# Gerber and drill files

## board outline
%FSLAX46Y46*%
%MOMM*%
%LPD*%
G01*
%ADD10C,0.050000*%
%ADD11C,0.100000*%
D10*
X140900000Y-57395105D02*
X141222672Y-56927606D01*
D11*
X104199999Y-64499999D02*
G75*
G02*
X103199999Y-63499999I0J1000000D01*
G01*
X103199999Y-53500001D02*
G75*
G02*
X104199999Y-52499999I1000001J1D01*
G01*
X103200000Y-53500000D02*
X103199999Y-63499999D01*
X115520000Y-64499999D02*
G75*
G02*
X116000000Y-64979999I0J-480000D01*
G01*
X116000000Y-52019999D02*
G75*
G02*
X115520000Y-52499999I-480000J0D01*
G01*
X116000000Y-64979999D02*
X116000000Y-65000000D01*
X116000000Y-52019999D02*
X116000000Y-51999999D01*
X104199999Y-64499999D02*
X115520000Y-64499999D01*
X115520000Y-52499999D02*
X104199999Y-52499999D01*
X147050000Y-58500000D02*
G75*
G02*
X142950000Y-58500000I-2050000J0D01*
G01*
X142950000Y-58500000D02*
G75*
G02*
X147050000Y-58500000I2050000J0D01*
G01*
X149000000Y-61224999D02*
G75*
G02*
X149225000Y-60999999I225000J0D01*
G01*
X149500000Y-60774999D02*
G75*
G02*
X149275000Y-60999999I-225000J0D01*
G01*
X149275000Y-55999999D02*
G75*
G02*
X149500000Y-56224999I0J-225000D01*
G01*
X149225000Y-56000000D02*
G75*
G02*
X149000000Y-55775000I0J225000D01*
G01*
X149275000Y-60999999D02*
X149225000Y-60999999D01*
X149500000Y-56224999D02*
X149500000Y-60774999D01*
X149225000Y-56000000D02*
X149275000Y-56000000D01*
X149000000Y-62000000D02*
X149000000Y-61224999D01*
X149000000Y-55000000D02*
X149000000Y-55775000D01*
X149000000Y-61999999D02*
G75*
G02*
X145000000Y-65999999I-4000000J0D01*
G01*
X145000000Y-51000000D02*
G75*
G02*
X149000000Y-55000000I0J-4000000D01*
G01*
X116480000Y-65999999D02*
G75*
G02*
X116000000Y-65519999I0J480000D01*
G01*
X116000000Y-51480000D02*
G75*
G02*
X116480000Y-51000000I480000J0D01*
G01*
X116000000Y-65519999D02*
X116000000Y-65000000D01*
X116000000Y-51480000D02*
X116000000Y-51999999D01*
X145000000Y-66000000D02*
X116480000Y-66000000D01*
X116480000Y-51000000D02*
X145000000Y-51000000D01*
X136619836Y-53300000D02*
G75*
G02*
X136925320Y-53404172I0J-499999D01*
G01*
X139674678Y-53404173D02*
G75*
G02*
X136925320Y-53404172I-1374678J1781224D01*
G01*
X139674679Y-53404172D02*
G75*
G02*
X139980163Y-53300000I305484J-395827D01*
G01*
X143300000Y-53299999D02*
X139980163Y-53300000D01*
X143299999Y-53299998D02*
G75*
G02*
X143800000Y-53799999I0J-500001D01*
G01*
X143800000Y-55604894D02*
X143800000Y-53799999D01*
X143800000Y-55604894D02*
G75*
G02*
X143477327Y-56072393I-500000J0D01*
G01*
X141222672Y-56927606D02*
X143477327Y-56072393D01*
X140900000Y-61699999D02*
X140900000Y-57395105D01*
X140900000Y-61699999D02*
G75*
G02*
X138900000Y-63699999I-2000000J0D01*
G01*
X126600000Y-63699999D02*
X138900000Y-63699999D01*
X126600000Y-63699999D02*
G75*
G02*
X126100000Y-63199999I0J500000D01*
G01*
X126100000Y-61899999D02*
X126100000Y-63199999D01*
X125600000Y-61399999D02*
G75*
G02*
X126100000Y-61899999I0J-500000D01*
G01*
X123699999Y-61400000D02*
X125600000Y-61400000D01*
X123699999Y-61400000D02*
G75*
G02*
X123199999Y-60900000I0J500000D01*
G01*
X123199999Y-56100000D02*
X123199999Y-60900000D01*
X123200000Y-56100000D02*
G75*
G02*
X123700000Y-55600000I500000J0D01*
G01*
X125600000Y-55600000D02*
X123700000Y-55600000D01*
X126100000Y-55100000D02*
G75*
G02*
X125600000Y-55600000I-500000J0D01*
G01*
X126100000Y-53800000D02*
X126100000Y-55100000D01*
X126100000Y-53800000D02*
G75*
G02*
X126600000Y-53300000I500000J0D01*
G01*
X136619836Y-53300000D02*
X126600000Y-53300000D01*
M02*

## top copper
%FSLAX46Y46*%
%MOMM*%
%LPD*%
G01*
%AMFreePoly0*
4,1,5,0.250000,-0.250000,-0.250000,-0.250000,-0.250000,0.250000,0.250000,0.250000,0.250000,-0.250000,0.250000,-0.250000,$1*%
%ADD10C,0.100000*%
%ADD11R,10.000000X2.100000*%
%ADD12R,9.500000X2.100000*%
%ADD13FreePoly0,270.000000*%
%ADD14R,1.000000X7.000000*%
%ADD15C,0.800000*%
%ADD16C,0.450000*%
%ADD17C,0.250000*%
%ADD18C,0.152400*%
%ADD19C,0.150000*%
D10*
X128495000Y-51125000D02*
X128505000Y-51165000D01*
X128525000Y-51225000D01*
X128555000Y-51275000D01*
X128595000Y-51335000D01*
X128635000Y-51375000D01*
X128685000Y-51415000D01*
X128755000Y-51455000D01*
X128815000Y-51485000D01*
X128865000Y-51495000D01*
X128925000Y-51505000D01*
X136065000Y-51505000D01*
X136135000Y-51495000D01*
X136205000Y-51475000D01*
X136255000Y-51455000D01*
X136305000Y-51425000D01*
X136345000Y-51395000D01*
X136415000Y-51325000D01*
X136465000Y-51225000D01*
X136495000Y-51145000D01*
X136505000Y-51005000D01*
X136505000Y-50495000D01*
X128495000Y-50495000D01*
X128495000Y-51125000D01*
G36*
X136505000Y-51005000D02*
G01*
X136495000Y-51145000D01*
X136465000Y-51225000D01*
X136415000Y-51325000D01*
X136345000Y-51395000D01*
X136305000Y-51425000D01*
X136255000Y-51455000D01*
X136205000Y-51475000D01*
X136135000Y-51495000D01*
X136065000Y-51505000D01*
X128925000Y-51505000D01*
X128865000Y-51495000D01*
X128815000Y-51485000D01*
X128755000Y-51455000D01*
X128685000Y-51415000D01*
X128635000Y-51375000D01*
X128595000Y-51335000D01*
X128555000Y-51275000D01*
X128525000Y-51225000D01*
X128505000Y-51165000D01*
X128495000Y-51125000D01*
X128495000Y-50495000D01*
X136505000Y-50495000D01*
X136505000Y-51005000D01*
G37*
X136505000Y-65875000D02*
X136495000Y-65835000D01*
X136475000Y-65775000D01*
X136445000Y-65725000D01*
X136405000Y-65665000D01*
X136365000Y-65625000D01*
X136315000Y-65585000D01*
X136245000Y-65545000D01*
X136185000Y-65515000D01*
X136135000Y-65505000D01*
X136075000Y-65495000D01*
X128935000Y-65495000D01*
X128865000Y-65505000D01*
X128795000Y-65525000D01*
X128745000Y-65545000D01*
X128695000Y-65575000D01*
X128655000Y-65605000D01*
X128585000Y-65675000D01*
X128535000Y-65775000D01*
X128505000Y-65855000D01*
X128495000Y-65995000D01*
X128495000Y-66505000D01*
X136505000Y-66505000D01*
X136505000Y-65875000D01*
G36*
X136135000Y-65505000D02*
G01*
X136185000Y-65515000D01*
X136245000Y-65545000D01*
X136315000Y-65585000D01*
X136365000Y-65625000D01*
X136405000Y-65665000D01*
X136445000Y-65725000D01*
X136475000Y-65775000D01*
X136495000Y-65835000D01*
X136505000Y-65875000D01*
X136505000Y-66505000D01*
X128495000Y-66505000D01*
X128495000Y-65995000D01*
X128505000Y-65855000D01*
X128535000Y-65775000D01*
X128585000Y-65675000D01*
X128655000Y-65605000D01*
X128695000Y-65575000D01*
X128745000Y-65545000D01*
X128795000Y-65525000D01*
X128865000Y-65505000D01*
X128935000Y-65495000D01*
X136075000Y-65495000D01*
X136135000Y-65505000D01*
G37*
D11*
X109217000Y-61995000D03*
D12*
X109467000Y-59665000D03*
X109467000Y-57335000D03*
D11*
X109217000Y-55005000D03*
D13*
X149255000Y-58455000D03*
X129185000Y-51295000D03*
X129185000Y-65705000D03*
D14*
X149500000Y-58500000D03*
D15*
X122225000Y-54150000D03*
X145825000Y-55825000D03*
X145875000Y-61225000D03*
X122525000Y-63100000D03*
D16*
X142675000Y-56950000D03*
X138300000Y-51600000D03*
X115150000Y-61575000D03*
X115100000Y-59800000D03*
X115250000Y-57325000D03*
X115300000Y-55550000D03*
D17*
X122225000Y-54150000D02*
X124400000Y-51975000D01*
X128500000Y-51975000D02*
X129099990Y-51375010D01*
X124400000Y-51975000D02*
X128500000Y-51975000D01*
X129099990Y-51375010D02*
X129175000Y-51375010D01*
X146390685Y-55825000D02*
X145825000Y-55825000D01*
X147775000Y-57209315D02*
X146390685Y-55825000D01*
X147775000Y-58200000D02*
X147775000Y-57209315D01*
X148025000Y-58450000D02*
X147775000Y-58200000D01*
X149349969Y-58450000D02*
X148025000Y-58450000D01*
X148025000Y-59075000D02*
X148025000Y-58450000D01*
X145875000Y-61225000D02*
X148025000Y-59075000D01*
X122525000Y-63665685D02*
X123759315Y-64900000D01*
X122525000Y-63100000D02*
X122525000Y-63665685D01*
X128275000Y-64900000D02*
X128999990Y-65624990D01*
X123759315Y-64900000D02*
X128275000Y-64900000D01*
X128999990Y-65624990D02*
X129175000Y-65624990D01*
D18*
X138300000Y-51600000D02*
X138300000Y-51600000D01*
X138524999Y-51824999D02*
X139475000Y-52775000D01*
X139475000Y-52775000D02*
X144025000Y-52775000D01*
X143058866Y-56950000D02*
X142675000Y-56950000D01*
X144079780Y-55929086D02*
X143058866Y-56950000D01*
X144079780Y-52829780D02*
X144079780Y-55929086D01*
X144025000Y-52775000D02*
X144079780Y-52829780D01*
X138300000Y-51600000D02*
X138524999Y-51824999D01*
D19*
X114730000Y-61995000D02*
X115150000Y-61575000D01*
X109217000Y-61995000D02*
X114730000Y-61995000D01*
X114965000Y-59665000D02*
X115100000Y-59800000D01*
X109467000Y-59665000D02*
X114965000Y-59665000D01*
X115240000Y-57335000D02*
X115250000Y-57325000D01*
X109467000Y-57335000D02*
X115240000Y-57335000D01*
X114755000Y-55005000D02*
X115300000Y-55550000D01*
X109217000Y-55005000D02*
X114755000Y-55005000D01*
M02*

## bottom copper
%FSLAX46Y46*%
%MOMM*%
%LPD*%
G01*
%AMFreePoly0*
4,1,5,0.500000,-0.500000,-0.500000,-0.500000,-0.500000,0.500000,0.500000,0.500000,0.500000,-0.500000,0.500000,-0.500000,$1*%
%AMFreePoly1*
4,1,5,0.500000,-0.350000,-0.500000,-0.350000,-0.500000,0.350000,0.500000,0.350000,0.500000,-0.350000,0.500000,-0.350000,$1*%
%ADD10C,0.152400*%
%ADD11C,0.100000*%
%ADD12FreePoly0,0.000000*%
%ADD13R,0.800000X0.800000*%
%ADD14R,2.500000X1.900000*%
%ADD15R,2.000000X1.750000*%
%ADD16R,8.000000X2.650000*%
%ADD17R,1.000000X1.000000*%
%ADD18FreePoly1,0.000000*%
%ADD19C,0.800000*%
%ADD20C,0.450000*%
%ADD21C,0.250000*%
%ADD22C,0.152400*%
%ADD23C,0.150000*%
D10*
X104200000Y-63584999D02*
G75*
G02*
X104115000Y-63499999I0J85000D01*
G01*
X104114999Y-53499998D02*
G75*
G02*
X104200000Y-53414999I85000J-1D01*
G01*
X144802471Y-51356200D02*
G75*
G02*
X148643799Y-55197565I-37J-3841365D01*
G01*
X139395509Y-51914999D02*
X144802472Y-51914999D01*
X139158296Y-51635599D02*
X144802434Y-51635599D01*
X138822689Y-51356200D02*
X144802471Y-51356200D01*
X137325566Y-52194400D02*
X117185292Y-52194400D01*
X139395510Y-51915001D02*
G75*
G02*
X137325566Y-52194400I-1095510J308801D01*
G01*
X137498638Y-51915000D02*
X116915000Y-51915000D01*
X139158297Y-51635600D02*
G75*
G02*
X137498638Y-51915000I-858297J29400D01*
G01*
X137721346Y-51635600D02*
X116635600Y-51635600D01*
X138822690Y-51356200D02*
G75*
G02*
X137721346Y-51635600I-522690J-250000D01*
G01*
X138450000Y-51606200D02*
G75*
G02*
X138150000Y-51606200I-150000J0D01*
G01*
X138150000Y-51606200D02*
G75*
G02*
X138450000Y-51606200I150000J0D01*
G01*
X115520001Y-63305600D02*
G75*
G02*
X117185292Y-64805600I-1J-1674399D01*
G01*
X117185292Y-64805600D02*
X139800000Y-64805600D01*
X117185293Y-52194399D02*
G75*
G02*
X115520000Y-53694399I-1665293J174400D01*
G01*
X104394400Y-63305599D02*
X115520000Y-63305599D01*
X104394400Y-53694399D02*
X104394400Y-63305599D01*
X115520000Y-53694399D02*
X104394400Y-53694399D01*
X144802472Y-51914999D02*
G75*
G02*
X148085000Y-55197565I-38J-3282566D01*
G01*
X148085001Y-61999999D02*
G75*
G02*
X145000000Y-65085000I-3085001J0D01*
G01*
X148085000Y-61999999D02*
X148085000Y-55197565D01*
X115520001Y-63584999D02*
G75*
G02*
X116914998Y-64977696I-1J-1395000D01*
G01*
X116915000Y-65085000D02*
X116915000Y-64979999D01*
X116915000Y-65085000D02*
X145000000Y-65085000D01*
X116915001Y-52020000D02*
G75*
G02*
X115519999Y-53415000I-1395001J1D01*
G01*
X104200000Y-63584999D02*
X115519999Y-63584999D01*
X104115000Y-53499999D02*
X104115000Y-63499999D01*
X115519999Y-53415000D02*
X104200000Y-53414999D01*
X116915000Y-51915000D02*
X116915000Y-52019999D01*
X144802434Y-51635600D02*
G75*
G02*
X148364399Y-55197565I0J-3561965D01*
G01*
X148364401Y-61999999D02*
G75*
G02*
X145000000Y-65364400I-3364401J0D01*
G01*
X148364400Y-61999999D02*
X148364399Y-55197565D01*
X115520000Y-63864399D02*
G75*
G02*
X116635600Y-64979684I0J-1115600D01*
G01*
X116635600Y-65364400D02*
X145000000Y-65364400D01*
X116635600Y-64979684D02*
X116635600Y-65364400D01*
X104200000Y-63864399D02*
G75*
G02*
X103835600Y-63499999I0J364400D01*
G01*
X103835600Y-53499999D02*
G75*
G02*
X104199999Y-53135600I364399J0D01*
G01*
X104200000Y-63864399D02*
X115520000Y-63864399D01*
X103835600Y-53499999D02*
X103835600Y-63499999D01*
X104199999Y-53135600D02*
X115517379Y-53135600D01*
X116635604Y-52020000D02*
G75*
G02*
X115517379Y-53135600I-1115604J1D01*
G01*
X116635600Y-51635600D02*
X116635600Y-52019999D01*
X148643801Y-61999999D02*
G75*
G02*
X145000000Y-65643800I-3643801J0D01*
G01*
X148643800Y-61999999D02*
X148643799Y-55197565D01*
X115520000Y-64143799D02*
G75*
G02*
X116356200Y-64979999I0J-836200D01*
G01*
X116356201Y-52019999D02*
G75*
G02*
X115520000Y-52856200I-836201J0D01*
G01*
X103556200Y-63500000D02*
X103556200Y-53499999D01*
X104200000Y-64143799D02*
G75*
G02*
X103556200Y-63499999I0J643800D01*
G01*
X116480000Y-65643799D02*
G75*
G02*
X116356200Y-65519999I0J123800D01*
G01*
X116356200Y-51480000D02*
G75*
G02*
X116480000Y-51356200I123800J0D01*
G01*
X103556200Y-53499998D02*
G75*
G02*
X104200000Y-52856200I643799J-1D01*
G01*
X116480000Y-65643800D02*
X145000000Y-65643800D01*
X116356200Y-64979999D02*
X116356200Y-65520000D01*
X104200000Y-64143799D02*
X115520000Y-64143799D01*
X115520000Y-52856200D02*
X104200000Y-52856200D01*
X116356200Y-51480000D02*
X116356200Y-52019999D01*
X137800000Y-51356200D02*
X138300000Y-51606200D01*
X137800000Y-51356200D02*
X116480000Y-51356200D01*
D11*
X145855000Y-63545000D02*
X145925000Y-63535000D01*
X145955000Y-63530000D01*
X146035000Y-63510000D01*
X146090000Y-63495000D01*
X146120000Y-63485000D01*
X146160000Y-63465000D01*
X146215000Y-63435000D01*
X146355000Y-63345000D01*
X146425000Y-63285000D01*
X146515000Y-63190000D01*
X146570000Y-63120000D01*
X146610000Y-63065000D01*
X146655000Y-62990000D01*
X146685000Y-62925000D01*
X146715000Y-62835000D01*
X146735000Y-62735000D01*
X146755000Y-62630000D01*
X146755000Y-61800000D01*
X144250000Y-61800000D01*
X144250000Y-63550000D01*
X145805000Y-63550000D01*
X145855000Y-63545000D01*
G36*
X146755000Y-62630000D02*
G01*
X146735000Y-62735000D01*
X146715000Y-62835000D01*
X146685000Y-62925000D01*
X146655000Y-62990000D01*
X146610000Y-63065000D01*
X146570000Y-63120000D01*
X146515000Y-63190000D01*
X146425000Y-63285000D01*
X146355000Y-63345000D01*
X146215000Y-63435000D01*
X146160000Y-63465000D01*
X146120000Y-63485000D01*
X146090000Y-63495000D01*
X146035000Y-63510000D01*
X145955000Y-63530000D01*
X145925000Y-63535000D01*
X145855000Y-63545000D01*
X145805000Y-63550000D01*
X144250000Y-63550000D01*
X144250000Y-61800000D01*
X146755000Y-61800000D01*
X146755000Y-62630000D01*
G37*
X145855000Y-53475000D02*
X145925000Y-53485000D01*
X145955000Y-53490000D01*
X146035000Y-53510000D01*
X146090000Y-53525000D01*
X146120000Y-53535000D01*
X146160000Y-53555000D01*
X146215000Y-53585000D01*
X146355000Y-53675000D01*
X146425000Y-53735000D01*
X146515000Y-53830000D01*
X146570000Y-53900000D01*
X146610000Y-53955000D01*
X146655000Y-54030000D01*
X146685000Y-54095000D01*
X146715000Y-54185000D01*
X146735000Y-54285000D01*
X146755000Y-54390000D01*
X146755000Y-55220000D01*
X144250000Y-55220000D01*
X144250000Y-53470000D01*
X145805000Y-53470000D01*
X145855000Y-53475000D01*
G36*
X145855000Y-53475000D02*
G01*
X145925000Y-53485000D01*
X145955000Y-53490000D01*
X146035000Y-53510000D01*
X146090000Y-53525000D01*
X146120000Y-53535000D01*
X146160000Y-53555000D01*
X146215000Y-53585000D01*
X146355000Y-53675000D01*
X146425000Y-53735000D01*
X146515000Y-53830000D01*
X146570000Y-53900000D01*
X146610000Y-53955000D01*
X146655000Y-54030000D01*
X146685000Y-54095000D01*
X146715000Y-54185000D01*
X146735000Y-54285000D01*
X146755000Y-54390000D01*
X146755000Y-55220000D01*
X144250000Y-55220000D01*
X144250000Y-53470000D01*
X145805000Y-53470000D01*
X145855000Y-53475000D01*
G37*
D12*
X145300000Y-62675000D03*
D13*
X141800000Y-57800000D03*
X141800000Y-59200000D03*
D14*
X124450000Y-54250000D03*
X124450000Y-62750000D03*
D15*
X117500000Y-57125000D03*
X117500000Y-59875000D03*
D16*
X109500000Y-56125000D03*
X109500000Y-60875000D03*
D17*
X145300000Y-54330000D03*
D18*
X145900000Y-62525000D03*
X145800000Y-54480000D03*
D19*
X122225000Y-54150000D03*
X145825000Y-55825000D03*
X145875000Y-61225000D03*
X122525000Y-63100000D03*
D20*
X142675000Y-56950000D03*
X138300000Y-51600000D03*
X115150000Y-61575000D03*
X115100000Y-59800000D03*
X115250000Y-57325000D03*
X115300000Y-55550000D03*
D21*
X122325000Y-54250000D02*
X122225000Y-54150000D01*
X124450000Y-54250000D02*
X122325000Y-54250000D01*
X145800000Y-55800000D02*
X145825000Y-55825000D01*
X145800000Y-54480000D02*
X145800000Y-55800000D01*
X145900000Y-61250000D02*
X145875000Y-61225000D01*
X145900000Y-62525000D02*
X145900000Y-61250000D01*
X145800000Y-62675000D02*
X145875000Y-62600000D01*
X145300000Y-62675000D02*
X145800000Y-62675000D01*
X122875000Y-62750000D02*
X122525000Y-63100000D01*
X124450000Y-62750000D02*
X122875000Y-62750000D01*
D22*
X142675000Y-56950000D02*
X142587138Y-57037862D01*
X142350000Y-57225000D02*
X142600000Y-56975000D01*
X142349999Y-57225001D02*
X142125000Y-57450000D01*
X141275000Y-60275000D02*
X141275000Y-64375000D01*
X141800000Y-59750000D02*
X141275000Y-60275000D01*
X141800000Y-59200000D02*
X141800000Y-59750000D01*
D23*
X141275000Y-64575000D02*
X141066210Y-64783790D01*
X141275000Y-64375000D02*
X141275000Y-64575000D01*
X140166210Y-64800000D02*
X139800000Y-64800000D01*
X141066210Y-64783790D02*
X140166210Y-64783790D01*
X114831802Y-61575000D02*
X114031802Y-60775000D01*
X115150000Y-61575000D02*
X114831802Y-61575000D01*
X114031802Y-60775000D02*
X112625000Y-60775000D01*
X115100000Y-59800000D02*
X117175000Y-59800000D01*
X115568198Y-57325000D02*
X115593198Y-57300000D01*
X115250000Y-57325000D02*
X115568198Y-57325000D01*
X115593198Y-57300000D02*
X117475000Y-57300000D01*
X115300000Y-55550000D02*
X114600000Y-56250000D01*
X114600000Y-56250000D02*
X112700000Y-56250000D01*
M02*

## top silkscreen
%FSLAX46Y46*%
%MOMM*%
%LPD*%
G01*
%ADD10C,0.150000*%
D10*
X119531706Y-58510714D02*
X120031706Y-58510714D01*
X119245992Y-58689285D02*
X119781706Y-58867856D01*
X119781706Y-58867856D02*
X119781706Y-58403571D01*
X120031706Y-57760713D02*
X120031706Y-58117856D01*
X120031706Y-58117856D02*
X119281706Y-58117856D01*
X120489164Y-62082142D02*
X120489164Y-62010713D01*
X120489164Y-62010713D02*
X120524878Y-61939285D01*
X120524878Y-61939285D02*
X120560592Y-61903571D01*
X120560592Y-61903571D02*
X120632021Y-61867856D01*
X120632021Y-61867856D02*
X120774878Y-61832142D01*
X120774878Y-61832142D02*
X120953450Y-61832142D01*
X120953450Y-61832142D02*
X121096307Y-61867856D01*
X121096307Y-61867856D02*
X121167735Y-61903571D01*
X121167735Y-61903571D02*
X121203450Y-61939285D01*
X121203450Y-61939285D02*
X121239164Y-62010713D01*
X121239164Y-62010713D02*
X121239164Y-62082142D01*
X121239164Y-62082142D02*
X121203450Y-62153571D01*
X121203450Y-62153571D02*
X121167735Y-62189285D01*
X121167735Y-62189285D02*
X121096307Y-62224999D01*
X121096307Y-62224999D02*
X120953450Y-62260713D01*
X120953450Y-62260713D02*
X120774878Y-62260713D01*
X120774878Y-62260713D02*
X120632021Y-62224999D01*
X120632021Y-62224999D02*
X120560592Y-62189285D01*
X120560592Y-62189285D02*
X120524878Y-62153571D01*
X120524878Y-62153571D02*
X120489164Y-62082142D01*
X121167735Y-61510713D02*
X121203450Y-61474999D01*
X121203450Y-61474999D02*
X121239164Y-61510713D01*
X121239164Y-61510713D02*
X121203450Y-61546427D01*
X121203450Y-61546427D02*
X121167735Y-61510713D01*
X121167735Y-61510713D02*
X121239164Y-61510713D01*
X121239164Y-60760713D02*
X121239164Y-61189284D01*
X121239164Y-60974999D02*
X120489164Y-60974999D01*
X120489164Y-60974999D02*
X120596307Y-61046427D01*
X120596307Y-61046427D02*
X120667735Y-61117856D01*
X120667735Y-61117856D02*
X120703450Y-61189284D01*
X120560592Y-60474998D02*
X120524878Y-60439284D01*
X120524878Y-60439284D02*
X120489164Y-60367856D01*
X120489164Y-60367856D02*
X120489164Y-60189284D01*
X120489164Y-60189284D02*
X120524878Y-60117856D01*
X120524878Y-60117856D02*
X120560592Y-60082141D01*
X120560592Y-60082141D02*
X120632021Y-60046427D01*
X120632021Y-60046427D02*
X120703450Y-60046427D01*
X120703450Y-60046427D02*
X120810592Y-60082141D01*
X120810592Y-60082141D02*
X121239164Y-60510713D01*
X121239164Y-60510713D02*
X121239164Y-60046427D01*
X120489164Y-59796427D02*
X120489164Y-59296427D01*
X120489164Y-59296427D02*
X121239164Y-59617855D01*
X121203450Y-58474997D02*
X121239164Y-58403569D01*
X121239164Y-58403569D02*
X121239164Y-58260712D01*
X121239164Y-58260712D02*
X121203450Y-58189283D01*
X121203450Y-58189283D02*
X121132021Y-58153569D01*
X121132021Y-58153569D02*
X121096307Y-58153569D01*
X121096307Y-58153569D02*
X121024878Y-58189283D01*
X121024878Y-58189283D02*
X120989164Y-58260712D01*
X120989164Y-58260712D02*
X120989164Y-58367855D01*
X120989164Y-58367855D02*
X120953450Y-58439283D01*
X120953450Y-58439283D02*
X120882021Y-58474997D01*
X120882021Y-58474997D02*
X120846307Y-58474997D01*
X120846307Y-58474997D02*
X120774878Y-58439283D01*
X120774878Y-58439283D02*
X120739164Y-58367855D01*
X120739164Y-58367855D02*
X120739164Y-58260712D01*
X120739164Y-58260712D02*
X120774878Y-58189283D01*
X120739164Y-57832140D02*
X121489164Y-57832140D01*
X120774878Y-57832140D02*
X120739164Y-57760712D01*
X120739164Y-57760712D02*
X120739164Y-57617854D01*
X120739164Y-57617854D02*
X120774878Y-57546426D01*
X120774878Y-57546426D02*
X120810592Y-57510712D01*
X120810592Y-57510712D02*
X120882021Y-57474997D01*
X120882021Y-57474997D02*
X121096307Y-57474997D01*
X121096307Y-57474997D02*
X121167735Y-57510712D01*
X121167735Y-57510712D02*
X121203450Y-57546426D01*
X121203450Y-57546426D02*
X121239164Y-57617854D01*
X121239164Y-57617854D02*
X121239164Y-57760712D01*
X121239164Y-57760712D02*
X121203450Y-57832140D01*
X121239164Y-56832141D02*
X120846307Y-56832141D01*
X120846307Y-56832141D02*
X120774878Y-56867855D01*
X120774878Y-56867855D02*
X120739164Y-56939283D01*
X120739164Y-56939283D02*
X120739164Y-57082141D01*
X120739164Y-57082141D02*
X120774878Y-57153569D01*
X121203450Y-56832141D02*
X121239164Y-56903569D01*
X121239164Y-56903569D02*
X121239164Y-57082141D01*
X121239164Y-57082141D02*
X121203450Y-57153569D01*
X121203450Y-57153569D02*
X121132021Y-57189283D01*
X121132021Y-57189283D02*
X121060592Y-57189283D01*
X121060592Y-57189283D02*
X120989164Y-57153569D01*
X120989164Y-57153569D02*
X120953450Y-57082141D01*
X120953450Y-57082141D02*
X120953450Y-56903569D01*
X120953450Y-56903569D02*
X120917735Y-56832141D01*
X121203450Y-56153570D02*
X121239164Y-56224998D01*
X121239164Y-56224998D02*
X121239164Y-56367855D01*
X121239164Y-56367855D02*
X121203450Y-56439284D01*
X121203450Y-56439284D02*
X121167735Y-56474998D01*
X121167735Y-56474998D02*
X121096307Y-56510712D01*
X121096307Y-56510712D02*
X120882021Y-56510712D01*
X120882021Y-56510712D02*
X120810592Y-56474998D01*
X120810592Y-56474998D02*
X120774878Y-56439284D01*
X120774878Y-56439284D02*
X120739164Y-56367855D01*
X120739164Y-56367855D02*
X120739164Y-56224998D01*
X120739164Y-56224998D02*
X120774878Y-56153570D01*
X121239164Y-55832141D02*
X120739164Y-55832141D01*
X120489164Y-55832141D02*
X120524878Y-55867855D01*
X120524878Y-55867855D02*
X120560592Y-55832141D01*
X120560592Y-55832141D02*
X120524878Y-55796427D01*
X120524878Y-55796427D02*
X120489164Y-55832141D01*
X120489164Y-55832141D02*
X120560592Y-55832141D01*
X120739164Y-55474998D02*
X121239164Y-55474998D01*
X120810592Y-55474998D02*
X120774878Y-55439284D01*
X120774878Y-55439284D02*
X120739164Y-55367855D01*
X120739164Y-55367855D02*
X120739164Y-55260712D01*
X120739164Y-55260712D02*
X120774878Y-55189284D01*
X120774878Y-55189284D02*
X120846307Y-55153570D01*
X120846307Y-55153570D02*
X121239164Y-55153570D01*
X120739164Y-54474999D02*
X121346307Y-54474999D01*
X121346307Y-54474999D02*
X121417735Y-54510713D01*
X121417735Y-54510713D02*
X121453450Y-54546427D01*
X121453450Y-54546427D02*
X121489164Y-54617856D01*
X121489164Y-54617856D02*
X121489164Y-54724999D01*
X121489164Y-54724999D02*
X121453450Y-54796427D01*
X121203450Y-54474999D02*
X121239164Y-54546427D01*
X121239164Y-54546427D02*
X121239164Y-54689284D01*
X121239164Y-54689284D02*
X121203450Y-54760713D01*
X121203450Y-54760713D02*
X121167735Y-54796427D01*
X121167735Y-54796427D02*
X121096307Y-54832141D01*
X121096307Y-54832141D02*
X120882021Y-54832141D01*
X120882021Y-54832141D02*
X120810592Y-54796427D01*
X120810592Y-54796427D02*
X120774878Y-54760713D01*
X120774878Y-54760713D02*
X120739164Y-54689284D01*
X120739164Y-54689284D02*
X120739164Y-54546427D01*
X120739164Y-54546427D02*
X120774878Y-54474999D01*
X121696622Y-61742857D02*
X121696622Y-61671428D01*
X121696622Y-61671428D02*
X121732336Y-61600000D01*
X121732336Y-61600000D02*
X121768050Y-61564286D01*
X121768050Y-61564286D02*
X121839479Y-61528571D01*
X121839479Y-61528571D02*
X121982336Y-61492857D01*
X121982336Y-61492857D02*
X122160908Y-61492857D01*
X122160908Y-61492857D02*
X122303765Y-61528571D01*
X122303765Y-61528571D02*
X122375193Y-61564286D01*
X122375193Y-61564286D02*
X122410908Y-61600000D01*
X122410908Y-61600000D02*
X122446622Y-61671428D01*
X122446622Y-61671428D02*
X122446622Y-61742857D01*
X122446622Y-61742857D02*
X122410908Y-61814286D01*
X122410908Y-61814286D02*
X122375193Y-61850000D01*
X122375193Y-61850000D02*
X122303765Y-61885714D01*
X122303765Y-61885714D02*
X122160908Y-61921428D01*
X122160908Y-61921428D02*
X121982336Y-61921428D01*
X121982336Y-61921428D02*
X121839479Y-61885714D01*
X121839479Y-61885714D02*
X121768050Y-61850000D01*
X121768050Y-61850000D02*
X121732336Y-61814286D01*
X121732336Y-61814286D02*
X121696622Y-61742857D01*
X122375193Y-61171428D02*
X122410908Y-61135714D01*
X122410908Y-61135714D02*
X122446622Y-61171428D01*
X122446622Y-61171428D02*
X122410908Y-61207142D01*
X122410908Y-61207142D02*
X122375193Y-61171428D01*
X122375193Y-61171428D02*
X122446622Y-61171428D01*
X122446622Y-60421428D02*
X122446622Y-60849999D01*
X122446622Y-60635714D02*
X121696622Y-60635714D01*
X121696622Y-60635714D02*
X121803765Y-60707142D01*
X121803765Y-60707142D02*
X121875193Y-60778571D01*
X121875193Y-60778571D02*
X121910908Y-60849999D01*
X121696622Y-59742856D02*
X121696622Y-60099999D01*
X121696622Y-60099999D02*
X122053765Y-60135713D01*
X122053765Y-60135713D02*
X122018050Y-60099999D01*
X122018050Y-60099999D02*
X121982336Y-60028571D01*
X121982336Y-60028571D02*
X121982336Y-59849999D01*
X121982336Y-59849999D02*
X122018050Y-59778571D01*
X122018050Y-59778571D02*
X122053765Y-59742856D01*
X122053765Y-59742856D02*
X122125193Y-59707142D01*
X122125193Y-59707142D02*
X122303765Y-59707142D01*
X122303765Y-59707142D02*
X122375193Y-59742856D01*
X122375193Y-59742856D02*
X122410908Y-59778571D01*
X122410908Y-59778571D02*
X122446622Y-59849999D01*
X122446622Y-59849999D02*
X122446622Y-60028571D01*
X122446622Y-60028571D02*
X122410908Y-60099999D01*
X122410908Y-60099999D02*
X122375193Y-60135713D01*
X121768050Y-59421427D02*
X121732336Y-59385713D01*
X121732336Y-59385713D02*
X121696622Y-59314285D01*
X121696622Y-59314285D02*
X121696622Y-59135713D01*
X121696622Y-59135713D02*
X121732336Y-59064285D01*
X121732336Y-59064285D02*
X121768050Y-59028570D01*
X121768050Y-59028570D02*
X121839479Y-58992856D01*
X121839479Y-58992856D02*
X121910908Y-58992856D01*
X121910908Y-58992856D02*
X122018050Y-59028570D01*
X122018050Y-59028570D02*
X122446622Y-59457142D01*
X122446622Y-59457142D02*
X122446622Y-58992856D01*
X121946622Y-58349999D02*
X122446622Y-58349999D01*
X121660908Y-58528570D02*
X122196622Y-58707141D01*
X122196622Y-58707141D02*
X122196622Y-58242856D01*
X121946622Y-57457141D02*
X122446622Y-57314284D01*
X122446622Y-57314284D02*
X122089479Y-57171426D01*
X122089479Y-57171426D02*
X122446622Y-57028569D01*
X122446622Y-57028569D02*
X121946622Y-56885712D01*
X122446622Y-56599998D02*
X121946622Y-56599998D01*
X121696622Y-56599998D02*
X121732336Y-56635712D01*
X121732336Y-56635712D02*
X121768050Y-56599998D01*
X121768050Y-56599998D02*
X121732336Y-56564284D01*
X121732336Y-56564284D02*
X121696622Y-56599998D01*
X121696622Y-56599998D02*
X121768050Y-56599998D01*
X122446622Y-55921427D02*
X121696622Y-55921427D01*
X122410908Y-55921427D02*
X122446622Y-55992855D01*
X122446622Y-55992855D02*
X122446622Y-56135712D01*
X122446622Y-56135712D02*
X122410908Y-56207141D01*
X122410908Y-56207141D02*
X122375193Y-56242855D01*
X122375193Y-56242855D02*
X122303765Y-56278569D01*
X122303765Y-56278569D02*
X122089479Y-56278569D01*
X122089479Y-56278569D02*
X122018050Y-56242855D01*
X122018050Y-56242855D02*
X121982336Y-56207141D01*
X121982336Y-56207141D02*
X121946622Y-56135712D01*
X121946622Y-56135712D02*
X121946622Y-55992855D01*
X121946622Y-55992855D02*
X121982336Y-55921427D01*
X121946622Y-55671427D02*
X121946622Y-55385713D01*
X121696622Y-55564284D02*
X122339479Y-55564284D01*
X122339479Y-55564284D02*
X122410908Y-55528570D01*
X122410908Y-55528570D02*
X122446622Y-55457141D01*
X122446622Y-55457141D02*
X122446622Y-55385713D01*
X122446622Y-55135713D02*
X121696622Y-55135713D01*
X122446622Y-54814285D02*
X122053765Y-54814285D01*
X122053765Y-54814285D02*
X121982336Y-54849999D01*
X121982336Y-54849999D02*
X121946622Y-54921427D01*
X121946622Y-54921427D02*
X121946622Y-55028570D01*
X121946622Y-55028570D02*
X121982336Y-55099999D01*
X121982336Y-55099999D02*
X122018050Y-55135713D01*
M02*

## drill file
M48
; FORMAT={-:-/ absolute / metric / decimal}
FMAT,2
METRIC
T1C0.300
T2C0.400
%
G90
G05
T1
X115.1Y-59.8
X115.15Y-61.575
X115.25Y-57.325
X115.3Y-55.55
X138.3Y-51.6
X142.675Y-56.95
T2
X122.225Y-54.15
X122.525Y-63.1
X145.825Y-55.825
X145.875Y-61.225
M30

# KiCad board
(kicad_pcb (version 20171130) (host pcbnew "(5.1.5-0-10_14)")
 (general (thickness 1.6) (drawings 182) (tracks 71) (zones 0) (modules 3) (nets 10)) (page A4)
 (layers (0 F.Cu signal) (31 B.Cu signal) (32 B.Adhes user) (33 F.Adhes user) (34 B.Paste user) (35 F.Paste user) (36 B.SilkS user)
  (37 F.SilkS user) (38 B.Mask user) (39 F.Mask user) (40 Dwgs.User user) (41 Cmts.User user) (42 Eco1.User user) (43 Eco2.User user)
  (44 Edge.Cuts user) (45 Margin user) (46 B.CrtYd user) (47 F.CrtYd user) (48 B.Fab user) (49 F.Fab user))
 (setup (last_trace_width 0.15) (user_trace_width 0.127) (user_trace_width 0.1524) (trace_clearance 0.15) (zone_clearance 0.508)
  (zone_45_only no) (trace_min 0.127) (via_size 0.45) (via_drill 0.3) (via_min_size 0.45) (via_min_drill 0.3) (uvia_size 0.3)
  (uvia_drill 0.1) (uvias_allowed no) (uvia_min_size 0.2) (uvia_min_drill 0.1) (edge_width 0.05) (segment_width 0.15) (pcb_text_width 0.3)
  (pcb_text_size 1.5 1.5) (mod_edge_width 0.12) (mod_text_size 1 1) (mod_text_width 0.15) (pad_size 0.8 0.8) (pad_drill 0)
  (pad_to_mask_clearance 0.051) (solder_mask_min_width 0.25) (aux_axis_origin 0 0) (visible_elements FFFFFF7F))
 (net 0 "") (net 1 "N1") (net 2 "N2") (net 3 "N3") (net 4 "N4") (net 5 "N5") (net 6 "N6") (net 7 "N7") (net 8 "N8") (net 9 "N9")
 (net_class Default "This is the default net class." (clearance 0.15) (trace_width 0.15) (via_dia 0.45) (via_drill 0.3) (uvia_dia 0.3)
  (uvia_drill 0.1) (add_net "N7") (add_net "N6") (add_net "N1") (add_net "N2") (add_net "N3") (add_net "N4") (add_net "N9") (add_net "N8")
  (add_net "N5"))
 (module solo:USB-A (layer F.Cu) (at 104.625 58.5)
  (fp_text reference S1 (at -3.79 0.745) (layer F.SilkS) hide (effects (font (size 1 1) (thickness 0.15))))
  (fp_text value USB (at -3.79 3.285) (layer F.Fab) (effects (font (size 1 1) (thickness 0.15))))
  (pad 1 smd rect (at 4.592 3.495) (size 10 2.1) (layers F.Cu F.Mask) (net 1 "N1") (solder_mask_margin 0.01))
  (pad 2 smd rect (at 4.842 1.165) (size 9.5 2.1) (layers F.Cu F.Mask) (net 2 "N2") (solder_mask_margin 0.01))
  (pad 3 smd rect (at 4.842 -1.165) (size 9.5 2.1) (layers F.Cu F.Mask) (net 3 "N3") (solder_mask_margin 0.01))
  (pad 4 smd rect (at 4.592 -3.495) (size 10 2.1) (layers F.Cu F.Mask) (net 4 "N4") (solder_mask_margin 0.01)))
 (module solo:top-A (layer B.Cu) (at 114.8 58.375)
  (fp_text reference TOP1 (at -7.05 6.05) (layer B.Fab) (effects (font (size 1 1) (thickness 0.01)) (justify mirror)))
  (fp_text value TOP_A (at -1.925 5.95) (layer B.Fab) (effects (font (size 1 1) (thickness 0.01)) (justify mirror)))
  (fp_poly
   (pts (xy 31.055 5.17) (xy 31.125 5.16) (xy 31.155 5.155) (xy 31.235 5.135) (xy 31.29 5.12) (xy 31.32 5.11) (xy 31.36 5.09)
    (xy 31.415 5.06) (xy 31.555 4.97) (xy 31.625 4.91) (xy 31.715 4.815) (xy 31.77 4.745) (xy 31.81 4.69) (xy 31.855 4.615) (xy 31.885 4.55)
    (xy 31.915 4.46) (xy 31.935 4.36) (xy 31.955 4.255) (xy 31.955 3.425) (xy 29.45 3.425) (xy 29.45 5.175) (xy 31.005 5.175))
   (layer B.Cu) (width 0.1))
  (fp_poly
   (pts (xy 31.055 -4.9) (xy 31.125 -4.89) (xy 31.155 -4.885) (xy 31.235 -4.865) (xy 31.29 -4.85) (xy 31.32 -4.84) (xy 31.36 -4.82)
    (xy 31.415 -4.79) (xy 31.555 -4.7) (xy 31.625 -4.64) (xy 31.715 -4.545) (xy 31.77 -4.475) (xy 31.81 -4.42) (xy 31.855 -4.345)
    (xy 31.885 -4.28) (xy 31.915 -4.19) (xy 31.935 -4.09) (xy 31.955 -3.985) (xy 31.955 -3.155) (xy 29.45 -3.155) (xy 29.45 -4.905)
    (xy 31.005 -4.905))
   (layer B.Cu) (width 0.1))
  (pad 9 smd custom (at 30.5 4.3) (size 1 1) (layers B.Cu B.Paste B.Mask) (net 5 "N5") (solder_paste_margin_ratio -0.05) (zone_connect 0)
   (options (clearance outline) (anchor rect)) (primitives))
  (pad 8 smd rect (at 27 -0.575) (size 0.8 0.8) (layers B.Cu B.Paste B.Mask) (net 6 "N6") (solder_paste_margin_ratio -0.2))
  (pad 7 smd rect (at 27 0.825) (size 0.8 0.8) (layers B.Cu B.Paste B.Mask) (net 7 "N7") (solder_paste_margin_ratio -0.2))
  (pad 6 smd rect (at 9.65 -4.125) (size 2.5 1.9) (layers B.Cu B.Paste B.Mask) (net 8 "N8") (solder_paste_margin_ratio -0.25))
  (pad 5 smd rect (at 9.65 4.375) (size 2.5 1.9) (layers B.Cu B.Paste B.Mask) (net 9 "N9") (solder_paste_margin_ratio -0.25))
  (pad 4 smd rect (at 2.7 -1.25) (size 2 1.75) (layers B.Cu B.Paste B.Mask) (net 3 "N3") (solder_paste_margin_ratio -0.25))
  (pad 3 smd rect (at 2.7 1.5) (size 2 1.75) (layers B.Cu B.Paste B.Mask) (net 2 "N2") (solder_paste_margin_ratio -0.25))
  (pad 2 smd rect (at -5.3 -2.25) (size 8 2.65) (layers B.Cu B.Paste B.Mask) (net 4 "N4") (solder_paste_margin_ratio -0.25))
  (pad 1 smd rect (at -5.3 2.5) (size 8 2.65) (layers B.Cu B.Paste B.Mask) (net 1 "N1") (solder_paste_margin_ratio -0.25))
  (pad 9 smd rect (at 30.5 -4.045) (size 1 1) (layers B.Cu B.Paste B.Mask) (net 5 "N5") (solder_paste_margin_ratio -0.05))
  (pad 9 smd custom (at 31.1 4.15) (size 1 0.7) (layers B.Cu B.Paste B.Mask) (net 5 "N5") (solder_paste_margin_ratio -0.05) (zone_connect 0)
   (options (clearance outline) (anchor rect)) (primitives))
  (pad 9 smd custom (at 31 -3.895) (size 1 0.7) (layers B.Cu B.Paste B.Mask) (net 5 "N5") (solder_paste_margin_ratio -0.05) (zone_connect 0)
   (options (clearance outline) (anchor rect)) (primitives)))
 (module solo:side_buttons (layer B.Cu) (at 149.525 58.075)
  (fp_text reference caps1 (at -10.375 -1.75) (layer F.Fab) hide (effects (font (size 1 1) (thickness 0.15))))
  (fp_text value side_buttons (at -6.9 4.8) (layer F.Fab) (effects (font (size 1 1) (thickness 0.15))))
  (fp_poly
   (pts (xy -21.03 -6.95) (xy -21.02 -6.91) (xy -21 -6.85) (xy -20.97 -6.8) (xy -20.93 -6.74) (xy -20.89 -6.7) (xy -20.84 -6.66)
    (xy -20.77 -6.62) (xy -20.71 -6.59) (xy -20.66 -6.58) (xy -20.6 -6.57) (xy -13.46 -6.57) (xy -13.39 -6.58) (xy -13.32 -6.6)
    (xy -13.27 -6.62) (xy -13.22 -6.65) (xy -13.18 -6.68) (xy -13.11 -6.75) (xy -13.06 -6.85) (xy -13.03 -6.93) (xy -13.02 -7.07)
    (xy -13.02 -7.58) (xy -21.03 -7.58))
   (layer F.Cu) (width 0.1))
  (fp_poly
   (pts (xy -13.02 7.8) (xy -13.03 7.76) (xy -13.05 7.7) (xy -13.08 7.65) (xy -13.12 7.59) (xy -13.16 7.55) (xy -13.21 7.51)
    (xy -13.28 7.47) (xy -13.34 7.44) (xy -13.39 7.43) (xy -13.45 7.42) (xy -20.59 7.42) (xy -20.66 7.43) (xy -20.73 7.45) (xy -20.78 7.47)
    (xy -20.83 7.5) (xy -20.87 7.53) (xy -20.94 7.6) (xy -20.99 7.7) (xy -21.02 7.78) (xy -21.03 7.92) (xy -21.03 8.43) (xy -13.02 8.43))
   (layer F.Cu) (width 0.1))
  (pad 3 smd custom (at -0.27 0.38 270) (size 0.5 0.5) (layers F.Cu) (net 5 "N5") (solder_mask_margin 0.01) (zone_connect 0)
   (options (clearance outline) (anchor rect)) (primitives))
  (pad 2 smd custom (at -20.34 -6.78 270) (size 0.5 0.5) (layers F.Cu) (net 8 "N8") (solder_mask_margin 0.01) (zone_connect 0)
   (options (clearance outline) (anchor rect)) (primitives))
  (pad 1 smd custom (at -20.34 7.63 270) (size 0.5 0.5) (layers F.Cu) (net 9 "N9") (solder_mask_margin 0.01) (zone_connect 0)
   (options (clearance outline) (anchor rect)) (primitives))
  (pad 3 smd rect (at -0.025 0.425 270) (size 7 1) (layers F.Cu F.Mask) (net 5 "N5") (solder_mask_margin 0.01)))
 (gr_arc (start 104.2 63.499999) (end 104.115 63.499999) (angle -90) (layer B.Cu) (width 0.1524))
 (gr_arc (start 104.199999 53.499999) (end 104.2 53.414999) (angle -90.00000003) (layer B.Cu) (width 0.1524))
 (gr_arc (start 144.802434 55.197565) (end 148.643799 55.197565) (angle -89.99945032) (layer B.Cu) (width 0.1524))
 (gr_line (start 139.395509 51.914999) (end 144.802472 51.914999) (layer B.Cu) (width 0.1524))
 (gr_line (start 139.158296 51.635599) (end 144.802434 51.635599) (layer B.Cu) (width 0.1524))
 (gr_line (start 138.822689 51.3562) (end 144.802471 51.3562) (layer B.Cu) (width 0.1524))
 (gr_line (start 137.325566 52.1944) (end 117.185292 52.1944) (layer B.Cu) (width 0.1524))
 (gr_arc (start 138.3 51.6062) (end 137.325566 52.1944) (angle -133.1414633) (layer B.Cu) (width 0.1524))
 (gr_line (start 137.498638 51.915) (end 116.915 51.915) (layer B.Cu) (width 0.1524))
 (gr_arc (start 138.3 51.6062) (end 137.498638 51.915) (angle -156.9642812) (layer B.Cu) (width 0.1524))
 (gr_line (start 137.721346 51.6356) (end 116.6356 51.6356) (layer B.Cu) (width 0.1524))
 (gr_arc (start 138.3 51.6062) (end 137.721346 51.6356) (angle -202.653015) (layer B.Cu) (width 0.1524))
 (gr_circle (center 138.3 51.6062) (end 138.45 51.6062) (layer B.Cu) (width 0.1524))
 (gr_arc (start 115.52 64.979999) (end 117.185292 64.8056) (angle -84.02141663) (layer B.Cu) (width 0.1524))
 (gr_line (start 117.185292 64.8056) (end 139.8 64.8056) (layer B.Cu) (width 0.1524))
 (gr_arc (start 115.52 52.019999) (end 115.52 53.694399) (angle -84.02141663) (layer B.Cu) (width 0.1524))
 (gr_line (start 104.3944 63.305599) (end 115.52 63.305599) (layer B.Cu) (width 0.1524))
 (gr_line (start 104.3944 53.694399) (end 104.3944 63.305599) (layer B.Cu) (width 0.1524))
 (gr_line (start 115.52 53.694399) (end 104.3944 53.694399) (layer B.Cu) (width 0.1524))
 (gr_arc (start 144.802434 55.197565) (end 148.085 55.197565) (angle -89.9993327) (layer B.Cu) (width 0.1524))
 (gr_arc (start 145 61.999999) (end 145 65.085) (angle -90) (layer B.Cu) (width 0.1524))
 (gr_line (start 148.085 61.999999) (end 148.085 55.197565) (layer B.Cu) (width 0.1524))
 (gr_arc (start 115.52 64.979999) (end 116.914998 64.977696) (angle -89.90537951) (layer B.Cu) (width 0.1524))
 (gr_line (start 116.915 65.085) (end 116.915 64.979999) (layer B.Cu) (width 0.1524))
 (gr_line (start 116.915 65.085) (end 145 65.085) (layer B.Cu) (width 0.1524))
 (gr_arc (start 115.52 52.019999) (end 115.519999 53.415) (angle -90) (layer B.Cu) (width 0.1524))
 (gr_line (start 104.2 63.584999) (end 115.519999 63.584999) (layer B.Cu) (width 0.1524))
 (gr_line (start 104.115 53.499999) (end 104.115 63.499999) (layer B.Cu) (width 0.1524))
 (gr_line (start 115.519999 53.415) (end 104.2 53.414999) (layer B.Cu) (width 0.1524))
 (gr_line (start 116.915 51.915) (end 116.915 52.019999) (layer B.Cu) (width 0.1524))
 (gr_arc (start 144.802434 55.197565) (end 148.364399 55.197565) (angle -90) (layer B.Cu) (width 0.1524))
 (gr_arc (start 145 61.999999) (end 145 65.3644) (angle -90) (layer B.Cu) (width 0.1524))
 (gr_line (start 148.3644 61.999999) (end 148.364399 55.197565) (layer B.Cu) (width 0.1524))
 (gr_arc (start 115.52 64.979999) (end 116.6356 64.979684) (angle -89.98381385) (layer B.Cu) (width 0.1524))
 (gr_line (start 116.6356 65.3644) (end 145 65.3644) (layer B.Cu) (width 0.1524))
 (gr_line (start 116.6356 64.979684) (end 116.6356 65.3644) (layer B.Cu) (width 0.1524))
 (gr_arc (start 104.2 63.499999) (end 103.8356 63.499999) (angle -90) (layer B.Cu) (width 0.1524))
 (gr_arc (start 104.199999 53.499999) (end 104.199999 53.1356) (angle -90) (layer B.Cu) (width 0.1524))
 (gr_line (start 104.2 63.864399) (end 115.52 63.864399) (layer B.Cu) (width 0.1524))
 (gr_line (start 103.8356 53.499999) (end 103.8356 63.499999) (layer B.Cu) (width 0.1524))
 (gr_line (start 104.199999 53.1356) (end 115.517379 53.1356) (layer B.Cu) (width 0.1524))
 (gr_arc (start 115.52 52.019999) (end 115.517379 53.1356) (angle -90.13456335) (layer B.Cu) (width 0.1524))
 (gr_line (start 116.6356 51.6356) (end 116.6356 52.019999) (layer B.Cu) (width 0.1524))
 (gr_arc (start 145 61.999999) (end 145 65.6438) (angle -90) (layer B.Cu) (width 0.1524))
 (gr_line (start 148.6438 61.999999) (end 148.643799 55.197565) (layer B.Cu) (width 0.1524))
 (gr_arc (start 115.52 64.979999) (end 116.3562 64.979999) (angle -90) (layer B.Cu) (width 0.1524))
 (gr_arc (start 115.52 52.019999) (end 115.52 52.8562) (angle -90) (layer B.Cu) (width 0.1524))
 (gr_line (start 103.5562 63.5) (end 103.5562 53.499999) (layer B.Cu) (width 0.1524))
 (gr_arc (start 104.2 63.499999) (end 103.5562 63.499999) (angle -90) (layer B.Cu) (width 0.1524))
 (gr_arc (start 116.48 65.519999) (end 116.3562 65.519999) (angle -90) (layer B.Cu) (width 0.1524))
 (gr_arc (start 116.48 51.48) (end 116.48 51.3562) (angle -90) (layer B.Cu) (width 0.1524))
 (gr_arc (start 104.199999 53.499999) (end 104.2 52.8562) (angle -90) (layer B.Cu) (width 0.1524))
 (gr_line (start 116.48 65.6438) (end 145 65.6438) (layer B.Cu) (width 0.1524))
 (gr_line (start 116.3562 64.979999) (end 116.3562 65.52) (layer B.Cu) (width 0.1524))
 (gr_line (start 104.2 64.143799) (end 115.52 64.143799) (layer B.Cu) (width 0.1524))
 (gr_line (start 115.52 52.8562) (end 104.2 52.8562) (layer B.Cu) (width 0.1524))
 (gr_line (start 116.3562 51.48) (end 116.3562 52.019999) (layer B.Cu) (width 0.1524))
 (gr_line (start 137.8 51.3562) (end 138.3 51.6062) (layer B.Cu) (width 0.1524))
 (gr_line (start 137.8 51.3562) (end 116.48 51.3562) (layer B.Cu) (width 0.1524))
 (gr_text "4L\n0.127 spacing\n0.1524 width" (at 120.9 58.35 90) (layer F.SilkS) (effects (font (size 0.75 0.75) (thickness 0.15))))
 (gr_line (start 140.9 57.395105) (end 141.222672 56.927606) (layer Edge.Cuts) (width 0.05))
 (gr_arc (start 104.199999 63.499999) (end 103.199999 63.499999) (angle -90) (layer Edge.Cuts) (width 0.1))
 (gr_arc (start 104.2 53.5) (end 104.199999 52.499999) (angle -90) (layer Edge.Cuts) (width 0.1))
 (gr_line (start 103.2 53.5) (end 103.199999 63.499999) (layer Edge.Cuts) (width 0.1))
 (gr_arc (start 115.52 64.979999) (end 116 64.979999) (angle -90) (layer Edge.Cuts) (width 0.1))
 (gr_arc (start 115.52 52.019999) (end 115.52 52.499999) (angle -90) (layer Edge.Cuts) (width 0.1))
 (gr_line (start 116 64.979999) (end 116 65) (layer Edge.Cuts) (width 0.1))
 (gr_line (start 116 52.019999) (end 116 51.999999) (layer Edge.Cuts) (width 0.1))
 (gr_line (start 104.199999 64.499999) (end 115.52 64.499999) (layer Edge.Cuts) (width 0.1))
 (gr_line (start 115.52 52.499999) (end 104.199999 52.499999) (layer Edge.Cuts) (width 0.1))
 (gr_circle (center 145 58.5) (end 147.05 58.5) (layer Edge.Cuts) (width 0.1))
 (gr_arc (start 149.225 61.224999) (end 149.225 60.999999) (angle -90) (layer Edge.Cuts) (width 0.1))
 (gr_arc (start 149.275 60.774999) (end 149.275 60.999999) (angle -90) (layer Edge.Cuts) (width 0.1))
 (gr_arc (start 149.275 56.224999) (end 149.5 56.224999) (angle -90) (layer Edge.Cuts) (width 0.1))
 (gr_arc (start 149.225 55.775) (end 149 55.775) (angle -90) (layer Edge.Cuts) (width 0.1))
 (gr_line (start 149.275 60.999999) (end 149.225 60.999999) (layer Edge.Cuts) (width 0.1))
 (gr_line (start 149.5 56.224999) (end 149.5 60.774999) (layer Edge.Cuts) (width 0.1))
 (gr_line (start 149.225 56) (end 149.275 56) (layer Edge.Cuts) (width 0.1))
 (gr_line (start 149 62) (end 149 61.224999) (layer Edge.Cuts) (width 0.1))
 (gr_line (start 149 55) (end 149 55.775) (layer Edge.Cuts) (width 0.1))
 (gr_arc (start 145 61.999999) (end 145 65.999999) (angle -90) (layer Edge.Cuts) (width 0.1))
 (gr_arc (start 145 55) (end 149 55) (angle -90) (layer Edge.Cuts) (width 0.1))
 (gr_arc (start 116.48 65.519999) (end 116 65.519999) (angle -90) (layer Edge.Cuts) (width 0.1))
 (gr_arc (start 116.48 51.48) (end 116.48 51) (angle -90) (layer Edge.Cuts) (width 0.1))
 (gr_line (start 116 65.519999) (end 116 65) (layer Edge.Cuts) (width 0.1))
 (gr_line (start 116 51.48) (end 116 51.999999) (layer Edge.Cuts) (width 0.1))
 (gr_line (start 145 66) (end 116.48 66) (layer Edge.Cuts) (width 0.1))
 (gr_line (start 116.48 51) (end 145 51) (layer Edge.Cuts) (width 0.1))
 (gr_arc (start 136.619836 53.799999) (end 136.92532 53.404172) (angle -37.6595652) (layer Edge.Cuts) (width 0.1))
 (gr_arc (start 138.3 51.622949) (end 136.92532 53.404172) (angle -75.31913041) (layer Edge.Cuts) (width 0.1))
 (gr_arc (start 139.980163 53.799999) (end 139.980163 53.3) (angle -37.6595652) (layer Edge.Cuts) (width 0.1))
 (gr_line (start 143.3 53.299999) (end 139.980163 53.3) (layer Edge.Cuts) (width 0.1))
 (gr_arc (start 143.299999 53.799999) (end 143.8 53.799999) (angle -90) (layer Edge.Cuts) (width 0.1))
 (gr_line (start 143.8 55.604894) (end 143.8 53.799999) (layer Edge.Cuts) (width 0.1))
 (gr_arc (start 143.3 55.604894) (end 143.477327 56.072393) (angle -69.22774532) (layer Edge.Cuts) (width 0.1))
 (gr_line (start 141.222672 56.927606) (end 143.477327 56.072393) (layer Edge.Cuts) (width 0.1))
 (gr_line (start 140.9 61.699999) (end 140.9 57.395105) (layer Edge.Cuts) (width 0.1))
 (gr_arc (start 138.9 61.699999) (end 138.9 63.699999) (angle -90) (layer Edge.Cuts) (width 0.1))
 (gr_line (start 126.6 63.699999) (end 138.9 63.699999) (layer Edge.Cuts) (width 0.1))
 (gr_arc (start 126.6 63.199999) (end 126.1 63.199999) (angle -90) (layer Edge.Cuts) (width 0.1))
 (gr_line (start 126.1 61.899999) (end 126.1 63.199999) (layer Edge.Cuts) (width 0.1))
 (gr_arc (start 125.6 61.899999) (end 126.1 61.899999) (angle -90) (layer Edge.Cuts) (width 0.1))
 (gr_line (start 123.699999 61.4) (end 125.6 61.4) (layer Edge.Cuts) (width 0.1))
 (gr_arc (start 123.699999 60.9) (end 123.199999 60.9) (angle -90) (layer Edge.Cuts) (width 0.1))
 (gr_line (start 123.199999 56.1) (end 123.199999 60.9) (layer Edge.Cuts) (width 0.1))
 (gr_arc (start 123.7 56.1) (end 123.7 55.6) (angle -90) (layer Edge.Cuts) (width 0.1))
 (gr_line (start 125.6 55.6) (end 123.7 55.6) (layer Edge.Cuts) (width 0.1))
 (gr_arc (start 125.6 55.1) (end 125.6 55.6) (angle -90) (layer Edge.Cuts) (width 0.1))
 (gr_line (start 126.1 53.8) (end 126.1 55.1) (layer Edge.Cuts) (width 0.1))
 (gr_arc (start 126.6 53.8) (end 126.6 53.3) (angle -90) (layer Edge.Cuts) (width 0.1))
 (gr_line (start 136.619836 53.3) (end 126.6 53.3) (layer Edge.Cuts) (width 0.1))
 (via (at 122.225 54.15) (size 0.8) (drill 0.4) (layers F.Cu B.Cu) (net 8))
 (segment (start 122.325 54.25) (end 122.225 54.15) (width 0.25) (layer B.Cu) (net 8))
 (segment (start 124.45 54.25) (end 122.325 54.25) (width 0.25) (layer B.Cu) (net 8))
 (segment (start 122.225 54.15) (end 124.4 51.975) (width 0.25) (layer F.Cu) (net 8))
 (segment (start 128.5 51.975) (end 129.09999 51.37501) (width 0.25) (layer F.Cu) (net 8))
 (segment (start 124.4 51.975) (end 128.5 51.975) (width 0.25) (layer F.Cu) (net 8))
 (segment (start 129.09999 51.37501) (end 129.175 51.37501) (width 0.25) (layer F.Cu) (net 8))
 (via (at 145.825 55.825) (size 0.8) (drill 0.4) (layers F.Cu B.Cu) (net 5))
 (segment (start 145.8 55.8) (end 145.825 55.825) (width 0.25) (layer B.Cu) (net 5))
 (segment (start 145.8 54.48) (end 145.8 55.8) (width 0.25) (layer B.Cu) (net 5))
 (segment (start 146.390685 55.825) (end 145.825 55.825) (width 0.25) (layer F.Cu) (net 5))
 (segment (start 147.775 57.209315) (end 146.390685 55.825) (width 0.25) (layer F.Cu) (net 5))
 (segment (start 147.775 58.2) (end 147.775 57.209315) (width 0.25) (layer F.Cu) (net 5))
 (segment (start 148.025 58.45) (end 147.775 58.2) (width 0.25) (layer F.Cu) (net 5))
 (segment (start 149.349969 58.45) (end 148.025 58.45) (width 0.25) (layer F.Cu) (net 5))
 (segment (start 145.9 61.25) (end 145.875 61.225) (width 0.25) (layer B.Cu) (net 5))
 (via (at 145.875 61.225) (size 0.8) (drill 0.4) (layers F.Cu B.Cu) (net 5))
 (segment (start 145.9 62.525) (end 145.9 61.25) (width 0.25) (layer B.Cu) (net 5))
 (segment (start 148.025 59.075) (end 148.025 58.45) (width 0.25) (layer F.Cu) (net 5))
 (segment (start 145.875 61.225) (end 148.025 59.075) (width 0.25) (layer F.Cu) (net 5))
 (segment (start 145.8 62.675) (end 145.875 62.6) (width 0.25) (layer B.Cu) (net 5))
 (segment (start 145.3 62.675) (end 145.8 62.675) (width 0.25) (layer B.Cu) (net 5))
 (via (at 122.525 63.1) (size 0.8) (drill 0.4) (layers F.Cu B.Cu) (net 9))
 (segment (start 122.875 62.75) (end 122.525 63.1) (width 0.25) (layer B.Cu) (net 9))
 (segment (start 124.45 62.75) (end 122.875 62.75) (width 0.25) (layer B.Cu) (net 9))
 (segment (start 122.525 63.665685) (end 123.759315 64.9) (width 0.25) (layer F.Cu) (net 9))
 (segment (start 122.525 63.1) (end 122.525 63.665685) (width 0.25) (layer F.Cu) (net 9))
 (segment (start 128.275 64.9) (end 128.99999 65.62499) (width 0.25) (layer F.Cu) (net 9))
 (segment (start 123.759315 64.9) (end 128.275 64.9) (width 0.25) (layer F.Cu) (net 9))
 (segment (start 128.99999 65.62499) (end 129.175 65.62499) (width 0.25) (layer F.Cu) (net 9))
 (segment (start 138.3 51.6) (end 138.3 51.6) (width 0.1524) (layer F.Cu) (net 6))
 (segment (start 138.524999 51.824999) (end 139.475 52.775) (width 0.1524) (layer F.Cu) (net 6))
 (segment (start 139.475 52.775) (end 144.025 52.775) (width 0.1524) (layer F.Cu) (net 6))
 (segment (start 143.058866 56.95) (end 142.675 56.95) (width 0.1524) (layer F.Cu) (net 6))
 (via (at 142.675 56.95) (size 0.45) (drill 0.3) (layers F.Cu B.Cu) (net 6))
 (segment (start 144.07978 55.929086) (end 143.058866 56.95) (width 0.1524) (layer F.Cu) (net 6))
 (segment (start 144.07978 52.82978) (end 144.07978 55.929086) (width 0.1524) (layer F.Cu) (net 6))
 (segment (start 144.025 52.775) (end 144.07978 52.82978) (width 0.1524) (layer F.Cu) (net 6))
 (segment (start 142.675 56.95) (end 142.587138 57.037862) (width 0.1524) (layer B.Cu) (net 6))
 (segment (start 142.35 57.225) (end 142.6 56.975) (width 0.1524) (layer B.Cu) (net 6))
 (segment (start 142.349999 57.225001) (end 142.125 57.45) (width 0.1524) (layer B.Cu) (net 6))
 (segment (start 138.3 51.6) (end 138.524999 51.824999) (width 0.1524) (layer F.Cu) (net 6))
 (via (at 138.3 51.6) (size 0.45) (drill 0.3) (layers F.Cu B.Cu) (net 6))
 (segment (start 141.275 60.275) (end 141.275 64.375) (width 0.1524) (layer B.Cu) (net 7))
 (segment (start 141.8 59.75) (end 141.275 60.275) (width 0.1524) (layer B.Cu) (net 7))
 (segment (start 141.8 59.2) (end 141.8 59.75) (width 0.1524) (layer B.Cu) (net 7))
 (segment (start 141.275 64.575) (end 141.06621 64.78379) (width 0.15) (layer B.Cu) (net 7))
 (segment (start 141.275 64.375) (end 141.275 64.575) (width 0.15) (layer B.Cu) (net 7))
 (segment (start 140.16621 64.8) (end 139.8 64.8) (width 0.15) (layer B.Cu) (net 7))
 (segment (start 141.06621 64.78379) (end 140.16621 64.78379) (width 0.15) (layer B.Cu) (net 7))
 (segment (start 114.73 61.995) (end 115.15 61.575) (width 0.15) (layer F.Cu) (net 1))
 (via (at 115.15 61.575) (size 0.45) (drill 0.3) (layers F.Cu B.Cu) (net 1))
 (segment (start 109.217 61.995) (end 114.73 61.995) (width 0.15) (layer F.Cu) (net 1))
 (segment (start 114.831802 61.575) (end 114.031802 60.775) (width 0.15) (layer B.Cu) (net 1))
 (segment (start 115.15 61.575) (end 114.831802 61.575) (width 0.15) (layer B.Cu) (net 1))
 (segment (start 114.031802 60.775) (end 112.625 60.775) (width 0.15) (layer B.Cu) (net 1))
 (via (at 115.1 59.8) (size 0.45) (drill 0.3) (layers F.Cu B.Cu) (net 2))
 (segment (start 114.965 59.665) (end 115.1 59.8) (width 0.15) (layer F.Cu) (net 2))
 (segment (start 109.467 59.665) (end 114.965 59.665) (width 0.15) (layer F.Cu) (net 2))
 (segment (start 115.1 59.8) (end 117.175 59.8) (width 0.15) (layer B.Cu) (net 2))
 (via (at 115.25 57.325) (size 0.45) (drill 0.3) (layers F.Cu B.Cu) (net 3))
 (segment (start 115.24 57.335) (end 115.25 57.325) (width 0.15) (layer F.Cu) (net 3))
 (segment (start 109.467 57.335) (end 115.24 57.335) (width 0.15) (layer F.Cu) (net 3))
 (segment (start 115.568198 57.325) (end 115.593198 57.3) (width 0.15) (layer B.Cu) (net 3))
 (segment (start 115.25 57.325) (end 115.568198 57.325) (width 0.15) (layer B.Cu) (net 3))
 (segment (start 115.593198 57.3) (end 117.475 57.3) (width 0.15) (layer B.Cu) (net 3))
 (via (at 115.3 55.55) (size 0.45) (drill 0.3) (layers F.Cu B.Cu) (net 4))
 (segment (start 114.755 55.005) (end 115.3 55.55) (width 0.15) (layer F.Cu) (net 4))
 (segment (start 109.217 55.005) (end 114.755 55.005) (width 0.15) (layer F.Cu) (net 4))
 (segment (start 115.3 55.55) (end 114.6 56.25) (width 0.15) (layer B.Cu) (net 4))
 (segment (start 114.6 56.25) (end 112.7 56.25) (width 0.15) (layer B.Cu) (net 4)))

